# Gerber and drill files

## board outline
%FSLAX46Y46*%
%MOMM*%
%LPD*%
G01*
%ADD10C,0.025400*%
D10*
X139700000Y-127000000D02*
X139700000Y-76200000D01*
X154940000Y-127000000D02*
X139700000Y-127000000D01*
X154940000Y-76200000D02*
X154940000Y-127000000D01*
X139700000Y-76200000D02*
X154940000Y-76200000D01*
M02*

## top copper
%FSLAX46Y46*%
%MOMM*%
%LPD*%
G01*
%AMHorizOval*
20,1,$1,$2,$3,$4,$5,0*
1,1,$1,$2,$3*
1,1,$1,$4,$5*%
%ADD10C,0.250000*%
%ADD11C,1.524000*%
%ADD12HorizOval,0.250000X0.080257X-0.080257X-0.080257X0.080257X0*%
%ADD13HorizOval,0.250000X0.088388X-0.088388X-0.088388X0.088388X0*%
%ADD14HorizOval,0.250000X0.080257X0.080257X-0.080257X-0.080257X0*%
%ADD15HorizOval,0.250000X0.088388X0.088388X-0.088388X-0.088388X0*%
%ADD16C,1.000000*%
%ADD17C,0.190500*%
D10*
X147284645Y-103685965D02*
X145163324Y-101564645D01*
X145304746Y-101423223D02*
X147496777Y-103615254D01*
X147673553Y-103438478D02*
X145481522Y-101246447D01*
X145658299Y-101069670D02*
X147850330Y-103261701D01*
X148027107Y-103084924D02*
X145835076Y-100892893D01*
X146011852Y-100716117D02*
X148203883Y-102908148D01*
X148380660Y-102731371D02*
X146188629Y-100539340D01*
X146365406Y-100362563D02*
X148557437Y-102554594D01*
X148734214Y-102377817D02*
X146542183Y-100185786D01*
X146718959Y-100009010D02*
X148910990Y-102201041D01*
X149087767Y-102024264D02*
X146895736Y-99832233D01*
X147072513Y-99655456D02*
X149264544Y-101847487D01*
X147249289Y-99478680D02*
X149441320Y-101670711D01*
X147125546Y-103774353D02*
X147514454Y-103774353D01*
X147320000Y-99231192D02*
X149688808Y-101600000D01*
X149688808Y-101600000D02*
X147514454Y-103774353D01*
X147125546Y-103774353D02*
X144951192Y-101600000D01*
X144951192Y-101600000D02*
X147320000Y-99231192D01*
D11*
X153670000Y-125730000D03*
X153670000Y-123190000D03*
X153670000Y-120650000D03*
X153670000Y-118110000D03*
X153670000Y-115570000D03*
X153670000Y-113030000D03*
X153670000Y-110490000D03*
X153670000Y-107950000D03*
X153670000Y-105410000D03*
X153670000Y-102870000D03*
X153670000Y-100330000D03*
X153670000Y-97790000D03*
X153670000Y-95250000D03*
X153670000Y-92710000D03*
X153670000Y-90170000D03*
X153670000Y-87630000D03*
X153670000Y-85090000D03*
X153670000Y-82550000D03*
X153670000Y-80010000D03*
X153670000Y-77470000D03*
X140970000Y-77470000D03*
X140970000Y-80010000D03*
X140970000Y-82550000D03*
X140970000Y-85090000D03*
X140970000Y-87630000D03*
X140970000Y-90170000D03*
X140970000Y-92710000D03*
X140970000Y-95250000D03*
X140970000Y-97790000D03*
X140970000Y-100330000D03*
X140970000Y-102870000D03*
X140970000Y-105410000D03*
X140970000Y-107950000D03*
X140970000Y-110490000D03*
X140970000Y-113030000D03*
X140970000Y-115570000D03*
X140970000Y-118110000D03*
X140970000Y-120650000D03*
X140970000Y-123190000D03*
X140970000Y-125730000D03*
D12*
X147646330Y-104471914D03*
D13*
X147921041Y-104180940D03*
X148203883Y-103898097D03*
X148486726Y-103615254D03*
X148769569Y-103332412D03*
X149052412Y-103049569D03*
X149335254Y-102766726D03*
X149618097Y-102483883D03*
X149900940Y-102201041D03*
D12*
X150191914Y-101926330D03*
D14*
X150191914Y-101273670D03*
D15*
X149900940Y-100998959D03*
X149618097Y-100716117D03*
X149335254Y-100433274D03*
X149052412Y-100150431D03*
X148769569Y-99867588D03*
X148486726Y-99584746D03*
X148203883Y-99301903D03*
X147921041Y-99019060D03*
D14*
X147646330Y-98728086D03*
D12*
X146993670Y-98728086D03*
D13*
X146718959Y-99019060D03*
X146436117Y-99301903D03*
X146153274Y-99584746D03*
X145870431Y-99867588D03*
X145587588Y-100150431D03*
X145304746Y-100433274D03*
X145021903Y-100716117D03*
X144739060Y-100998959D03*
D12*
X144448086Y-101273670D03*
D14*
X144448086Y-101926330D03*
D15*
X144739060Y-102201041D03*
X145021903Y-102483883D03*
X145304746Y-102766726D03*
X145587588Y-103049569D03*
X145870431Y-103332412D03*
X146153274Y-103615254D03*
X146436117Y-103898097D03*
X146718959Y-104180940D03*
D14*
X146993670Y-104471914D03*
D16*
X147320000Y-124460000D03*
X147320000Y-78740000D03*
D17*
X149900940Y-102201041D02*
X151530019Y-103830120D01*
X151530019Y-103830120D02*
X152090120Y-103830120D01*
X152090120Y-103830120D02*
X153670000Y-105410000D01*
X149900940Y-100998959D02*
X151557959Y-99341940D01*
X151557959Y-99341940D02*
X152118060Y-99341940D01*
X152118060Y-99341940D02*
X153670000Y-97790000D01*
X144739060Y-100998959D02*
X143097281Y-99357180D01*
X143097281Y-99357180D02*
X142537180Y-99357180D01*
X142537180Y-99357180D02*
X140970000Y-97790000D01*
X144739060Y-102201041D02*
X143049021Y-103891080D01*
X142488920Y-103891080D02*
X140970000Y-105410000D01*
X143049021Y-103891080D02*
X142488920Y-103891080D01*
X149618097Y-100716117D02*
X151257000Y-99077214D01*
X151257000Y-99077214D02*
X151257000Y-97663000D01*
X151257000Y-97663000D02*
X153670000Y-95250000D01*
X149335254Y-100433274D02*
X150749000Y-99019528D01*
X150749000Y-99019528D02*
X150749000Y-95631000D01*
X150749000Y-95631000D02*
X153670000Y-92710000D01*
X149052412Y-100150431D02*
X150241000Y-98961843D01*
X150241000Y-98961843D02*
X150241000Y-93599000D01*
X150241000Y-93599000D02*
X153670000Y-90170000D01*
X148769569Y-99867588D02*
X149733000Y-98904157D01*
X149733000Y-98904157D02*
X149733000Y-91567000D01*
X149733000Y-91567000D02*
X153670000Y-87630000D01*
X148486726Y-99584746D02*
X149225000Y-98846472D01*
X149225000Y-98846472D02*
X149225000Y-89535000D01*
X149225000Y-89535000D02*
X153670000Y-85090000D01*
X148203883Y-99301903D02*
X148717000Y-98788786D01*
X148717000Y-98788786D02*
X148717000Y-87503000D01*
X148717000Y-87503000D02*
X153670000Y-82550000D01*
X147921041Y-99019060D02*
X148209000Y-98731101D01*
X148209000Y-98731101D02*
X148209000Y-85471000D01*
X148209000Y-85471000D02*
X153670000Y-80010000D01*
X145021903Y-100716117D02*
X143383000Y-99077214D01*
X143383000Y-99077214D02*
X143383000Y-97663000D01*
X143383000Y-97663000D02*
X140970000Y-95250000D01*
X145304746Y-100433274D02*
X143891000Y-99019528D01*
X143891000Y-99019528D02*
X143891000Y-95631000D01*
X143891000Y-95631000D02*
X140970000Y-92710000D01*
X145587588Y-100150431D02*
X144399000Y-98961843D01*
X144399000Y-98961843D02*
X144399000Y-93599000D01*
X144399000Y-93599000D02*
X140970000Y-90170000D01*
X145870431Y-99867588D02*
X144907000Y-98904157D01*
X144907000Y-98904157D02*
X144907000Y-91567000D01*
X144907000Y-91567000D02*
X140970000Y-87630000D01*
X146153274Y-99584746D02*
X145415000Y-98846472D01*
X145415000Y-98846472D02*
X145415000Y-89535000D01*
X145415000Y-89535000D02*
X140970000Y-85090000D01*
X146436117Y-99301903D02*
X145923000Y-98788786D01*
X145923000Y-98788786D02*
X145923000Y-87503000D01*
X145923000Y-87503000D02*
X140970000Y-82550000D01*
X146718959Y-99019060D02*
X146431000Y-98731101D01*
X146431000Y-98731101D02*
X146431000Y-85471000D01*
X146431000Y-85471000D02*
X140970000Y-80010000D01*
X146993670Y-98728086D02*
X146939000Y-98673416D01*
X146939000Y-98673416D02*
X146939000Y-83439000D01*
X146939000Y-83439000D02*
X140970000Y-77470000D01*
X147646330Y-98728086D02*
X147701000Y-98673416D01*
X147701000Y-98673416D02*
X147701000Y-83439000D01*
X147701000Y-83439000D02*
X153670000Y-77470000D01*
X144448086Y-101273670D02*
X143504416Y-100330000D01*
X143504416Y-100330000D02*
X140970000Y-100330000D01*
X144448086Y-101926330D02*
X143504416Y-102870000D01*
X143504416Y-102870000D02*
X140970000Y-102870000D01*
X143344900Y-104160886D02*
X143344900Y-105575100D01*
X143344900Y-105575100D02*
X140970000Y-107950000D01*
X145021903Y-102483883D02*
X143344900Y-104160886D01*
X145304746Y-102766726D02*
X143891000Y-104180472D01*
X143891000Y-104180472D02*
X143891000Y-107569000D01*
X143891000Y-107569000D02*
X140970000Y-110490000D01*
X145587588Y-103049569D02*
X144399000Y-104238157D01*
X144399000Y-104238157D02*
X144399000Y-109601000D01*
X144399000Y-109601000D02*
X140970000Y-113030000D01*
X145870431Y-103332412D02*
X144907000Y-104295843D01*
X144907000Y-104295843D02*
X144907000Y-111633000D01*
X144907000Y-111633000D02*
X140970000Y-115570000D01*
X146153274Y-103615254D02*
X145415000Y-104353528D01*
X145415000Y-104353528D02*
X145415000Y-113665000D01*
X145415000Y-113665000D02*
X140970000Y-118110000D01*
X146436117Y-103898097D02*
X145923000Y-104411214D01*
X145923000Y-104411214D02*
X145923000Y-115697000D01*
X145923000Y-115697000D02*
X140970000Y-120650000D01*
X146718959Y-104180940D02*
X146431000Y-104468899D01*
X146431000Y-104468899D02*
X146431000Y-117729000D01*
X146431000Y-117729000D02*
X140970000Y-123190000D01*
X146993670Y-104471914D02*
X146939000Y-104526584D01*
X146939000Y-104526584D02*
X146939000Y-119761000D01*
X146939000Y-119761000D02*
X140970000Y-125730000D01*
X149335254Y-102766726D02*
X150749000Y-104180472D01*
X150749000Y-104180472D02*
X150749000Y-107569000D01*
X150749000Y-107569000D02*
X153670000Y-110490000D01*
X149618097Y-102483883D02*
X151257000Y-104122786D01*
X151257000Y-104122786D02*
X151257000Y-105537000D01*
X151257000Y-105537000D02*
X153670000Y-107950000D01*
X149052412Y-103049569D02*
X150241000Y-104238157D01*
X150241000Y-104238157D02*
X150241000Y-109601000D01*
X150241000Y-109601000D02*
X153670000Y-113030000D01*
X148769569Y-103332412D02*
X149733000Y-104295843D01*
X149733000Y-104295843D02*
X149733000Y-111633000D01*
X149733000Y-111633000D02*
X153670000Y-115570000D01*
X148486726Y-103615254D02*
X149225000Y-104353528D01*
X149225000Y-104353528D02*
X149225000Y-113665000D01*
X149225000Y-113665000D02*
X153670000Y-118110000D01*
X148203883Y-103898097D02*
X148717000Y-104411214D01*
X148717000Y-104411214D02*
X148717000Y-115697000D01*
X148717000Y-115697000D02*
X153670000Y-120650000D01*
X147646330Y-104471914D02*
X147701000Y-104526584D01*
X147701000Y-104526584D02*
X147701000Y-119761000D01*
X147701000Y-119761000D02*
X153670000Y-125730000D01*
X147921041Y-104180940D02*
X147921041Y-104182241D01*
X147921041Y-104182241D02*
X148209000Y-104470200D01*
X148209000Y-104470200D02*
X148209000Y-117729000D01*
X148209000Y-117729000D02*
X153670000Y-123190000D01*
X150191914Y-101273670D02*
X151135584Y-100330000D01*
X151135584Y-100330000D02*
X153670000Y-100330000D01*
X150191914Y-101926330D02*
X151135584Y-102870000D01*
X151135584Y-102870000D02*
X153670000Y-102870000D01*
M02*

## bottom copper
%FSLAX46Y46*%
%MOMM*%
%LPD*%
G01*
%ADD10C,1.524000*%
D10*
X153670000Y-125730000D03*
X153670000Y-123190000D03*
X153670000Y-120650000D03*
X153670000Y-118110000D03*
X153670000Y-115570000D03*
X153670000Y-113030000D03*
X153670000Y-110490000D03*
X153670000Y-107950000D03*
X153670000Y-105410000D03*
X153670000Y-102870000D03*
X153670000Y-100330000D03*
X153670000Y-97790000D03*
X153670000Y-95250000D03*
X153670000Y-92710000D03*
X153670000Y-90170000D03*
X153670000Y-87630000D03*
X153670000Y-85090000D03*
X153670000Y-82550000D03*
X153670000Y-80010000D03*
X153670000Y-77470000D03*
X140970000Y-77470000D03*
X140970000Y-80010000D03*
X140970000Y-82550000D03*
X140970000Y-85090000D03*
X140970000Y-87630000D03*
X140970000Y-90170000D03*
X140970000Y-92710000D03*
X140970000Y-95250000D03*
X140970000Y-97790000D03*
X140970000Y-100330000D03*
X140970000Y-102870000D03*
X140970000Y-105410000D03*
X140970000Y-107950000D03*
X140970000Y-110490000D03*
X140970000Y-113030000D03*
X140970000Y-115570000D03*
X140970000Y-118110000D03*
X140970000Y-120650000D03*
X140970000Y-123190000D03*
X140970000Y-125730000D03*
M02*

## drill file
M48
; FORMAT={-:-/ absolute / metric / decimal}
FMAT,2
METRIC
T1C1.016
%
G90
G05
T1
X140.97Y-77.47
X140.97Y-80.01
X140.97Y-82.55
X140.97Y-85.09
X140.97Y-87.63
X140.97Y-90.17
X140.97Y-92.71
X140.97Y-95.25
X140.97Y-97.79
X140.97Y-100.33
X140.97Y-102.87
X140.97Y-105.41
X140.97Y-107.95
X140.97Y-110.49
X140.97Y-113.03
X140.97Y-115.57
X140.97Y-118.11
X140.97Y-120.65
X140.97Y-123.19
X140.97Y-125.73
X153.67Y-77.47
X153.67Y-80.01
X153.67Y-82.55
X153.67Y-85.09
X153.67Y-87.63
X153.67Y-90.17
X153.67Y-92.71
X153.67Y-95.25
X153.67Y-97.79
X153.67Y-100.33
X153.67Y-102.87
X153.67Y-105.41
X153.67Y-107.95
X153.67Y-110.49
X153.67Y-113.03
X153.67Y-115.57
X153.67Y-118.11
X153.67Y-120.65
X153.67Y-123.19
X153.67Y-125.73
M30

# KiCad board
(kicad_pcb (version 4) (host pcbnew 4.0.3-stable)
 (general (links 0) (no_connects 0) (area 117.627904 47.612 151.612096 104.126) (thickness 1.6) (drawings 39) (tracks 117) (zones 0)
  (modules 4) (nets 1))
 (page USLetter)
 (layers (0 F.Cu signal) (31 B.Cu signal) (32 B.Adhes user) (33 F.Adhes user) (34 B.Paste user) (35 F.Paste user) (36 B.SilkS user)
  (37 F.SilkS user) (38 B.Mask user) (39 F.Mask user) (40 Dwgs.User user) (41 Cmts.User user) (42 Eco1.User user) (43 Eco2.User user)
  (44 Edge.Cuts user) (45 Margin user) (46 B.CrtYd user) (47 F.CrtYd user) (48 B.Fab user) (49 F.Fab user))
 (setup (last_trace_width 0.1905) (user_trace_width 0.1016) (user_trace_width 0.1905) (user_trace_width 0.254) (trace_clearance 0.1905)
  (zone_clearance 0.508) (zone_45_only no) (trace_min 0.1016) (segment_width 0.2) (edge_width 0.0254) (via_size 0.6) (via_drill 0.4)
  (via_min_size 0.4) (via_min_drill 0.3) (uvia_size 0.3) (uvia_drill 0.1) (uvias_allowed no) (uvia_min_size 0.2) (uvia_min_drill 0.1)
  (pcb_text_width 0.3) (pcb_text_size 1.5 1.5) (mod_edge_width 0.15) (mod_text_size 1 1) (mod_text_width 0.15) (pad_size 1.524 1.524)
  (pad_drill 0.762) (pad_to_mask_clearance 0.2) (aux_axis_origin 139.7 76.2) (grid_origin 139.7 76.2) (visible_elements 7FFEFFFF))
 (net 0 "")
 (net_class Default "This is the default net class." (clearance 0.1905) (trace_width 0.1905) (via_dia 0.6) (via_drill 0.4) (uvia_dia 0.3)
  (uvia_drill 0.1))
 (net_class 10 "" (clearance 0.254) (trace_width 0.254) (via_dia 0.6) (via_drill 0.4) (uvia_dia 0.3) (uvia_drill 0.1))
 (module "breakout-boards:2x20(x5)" (layer F.Cu) (at 147.32 101.6)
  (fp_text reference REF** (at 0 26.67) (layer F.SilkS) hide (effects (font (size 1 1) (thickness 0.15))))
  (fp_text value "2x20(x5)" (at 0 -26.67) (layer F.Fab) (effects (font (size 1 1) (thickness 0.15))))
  (pad 1 thru_hole circle (at 6.35 24.13) (size 1.524 1.524) (drill 1.016) (layers *.Cu *.Mask))
  (pad 2 thru_hole circle (at 6.35 21.59) (size 1.524 1.524) (drill 1.016) (layers *.Cu *.Mask))
  (pad 3 thru_hole circle (at 6.35 19.05) (size 1.524 1.524) (drill 1.016) (layers *.Cu *.Mask))
  (pad 4 thru_hole circle (at 6.35 16.51) (size 1.524 1.524) (drill 1.016) (layers *.Cu *.Mask))
  (pad 5 thru_hole circle (at 6.35 13.97) (size 1.524 1.524) (drill 1.016) (layers *.Cu *.Mask))
  (pad 6 thru_hole circle (at 6.35 11.43) (size 1.524 1.524) (drill 1.016) (layers *.Cu *.Mask))
  (pad 7 thru_hole circle (at 6.35 8.89) (size 1.524 1.524) (drill 1.016) (layers *.Cu *.Mask))
  (pad 8 thru_hole circle (at 6.35 6.35) (size 1.524 1.524) (drill 1.016) (layers *.Cu *.Mask))
  (pad 9 thru_hole circle (at 6.35 3.81) (size 1.524 1.524) (drill 1.016) (layers *.Cu *.Mask))
  (pad 10 thru_hole circle (at 6.35 1.27) (size 1.524 1.524) (drill 1.016) (layers *.Cu *.Mask))
  (pad 11 thru_hole circle (at 6.35 -1.27) (size 1.524 1.524) (drill 1.016) (layers *.Cu *.Mask))
  (pad 12 thru_hole circle (at 6.35 -3.81) (size 1.524 1.524) (drill 1.016) (layers *.Cu *.Mask))
  (pad 13 thru_hole circle (at 6.35 -6.35) (size 1.524 1.524) (drill 1.016) (layers *.Cu *.Mask))
  (pad 14 thru_hole circle (at 6.35 -8.89) (size 1.524 1.524) (drill 1.016) (layers *.Cu *.Mask))
  (pad 15 thru_hole circle (at 6.35 -11.43) (size 1.524 1.524) (drill 1.016) (layers *.Cu *.Mask))
  (pad 16 thru_hole circle (at 6.35 -13.97) (size 1.524 1.524) (drill 1.016) (layers *.Cu *.Mask))
  (pad 17 thru_hole circle (at 6.35 -16.51) (size 1.524 1.524) (drill 1.016) (layers *.Cu *.Mask))
  (pad 18 thru_hole circle (at 6.35 -19.05) (size 1.524 1.524) (drill 1.016) (layers *.Cu *.Mask))
  (pad 19 thru_hole circle (at 6.35 -21.59) (size 1.524 1.524) (drill 1.016) (layers *.Cu *.Mask))
  (pad 20 thru_hole circle (at 6.35 -24.13) (size 1.524 1.524) (drill 1.016) (layers *.Cu *.Mask))
  (pad 21 thru_hole circle (at -6.35 -24.13) (size 1.524 1.524) (drill 1.016) (layers *.Cu *.Mask))
  (pad 22 thru_hole circle (at -6.35 -21.59) (size 1.524 1.524) (drill 1.016) (layers *.Cu *.Mask))
  (pad 23 thru_hole circle (at -6.35 -19.05) (size 1.524 1.524) (drill 1.016) (layers *.Cu *.Mask))
  (pad 24 thru_hole circle (at -6.35 -16.51) (size 1.524 1.524) (drill 1.016) (layers *.Cu *.Mask))
  (pad 25 thru_hole circle (at -6.35 -13.97) (size 1.524 1.524) (drill 1.016) (layers *.Cu *.Mask))
  (pad 26 thru_hole circle (at -6.35 -11.43) (size 1.524 1.524) (drill 1.016) (layers *.Cu *.Mask))
  (pad 27 thru_hole circle (at -6.35 -8.89) (size 1.524 1.524) (drill 1.016) (layers *.Cu *.Mask))
  (pad 28 thru_hole circle (at -6.35 -6.35) (size 1.524 1.524) (drill 1.016) (layers *.Cu *.Mask))
  (pad 29 thru_hole circle (at -6.35 -3.81) (size 1.524 1.524) (drill 1.016) (layers *.Cu *.Mask))
  (pad 30 thru_hole circle (at -6.35 -1.27) (size 1.524 1.524) (drill 1.016) (layers *.Cu *.Mask))
  (pad 31 thru_hole circle (at -6.35 1.27) (size 1.524 1.524) (drill 1.016) (layers *.Cu *.Mask))
  (pad 32 thru_hole circle (at -6.35 3.81) (size 1.524 1.524) (drill 1.016) (layers *.Cu *.Mask))
  (pad 33 thru_hole circle (at -6.35 6.35) (size 1.524 1.524) (drill 1.016) (layers *.Cu *.Mask))
  (pad 34 thru_hole circle (at -6.35 8.89) (size 1.524 1.524) (drill 1.016) (layers *.Cu *.Mask))
  (pad 35 thru_hole circle (at -6.35 11.43) (size 1.524 1.524) (drill 1.016) (layers *.Cu *.Mask))
  (pad 36 thru_hole circle (at -6.35 13.97) (size 1.524 1.524) (drill 1.016) (layers *.Cu *.Mask))
  (pad 37 thru_hole circle (at -6.35 16.51) (size 1.524 1.524) (drill 1.016) (layers *.Cu *.Mask))
  (pad 38 thru_hole circle (at -6.35 19.05) (size 1.524 1.524) (drill 1.016) (layers *.Cu *.Mask))
  (pad 39 thru_hole circle (at -6.35 21.59) (size 1.524 1.524) (drill 1.016) (layers *.Cu *.Mask))
  (pad 40 thru_hole circle (at -6.35 24.13) (size 1.524 1.524) (drill 1.016) (layers *.Cu *.Mask)))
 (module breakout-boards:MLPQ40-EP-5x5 (layer F.Cu) (at 147.32 101.6 315)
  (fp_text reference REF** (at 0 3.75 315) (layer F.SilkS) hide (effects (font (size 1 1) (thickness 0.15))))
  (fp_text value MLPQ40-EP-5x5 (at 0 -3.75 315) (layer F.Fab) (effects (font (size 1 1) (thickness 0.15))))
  (fp_line (start 1.45 1.5) (end -1.55 1.5) (layer F.Cu) (width 0.25))
  (fp_line (start -1.55 1.3) (end 1.55 1.3) (layer F.Cu) (width 0.25))
  (fp_line (start 1.55 1.05) (end -1.55 1.05) (layer F.Cu) (width 0.25))
  (fp_line (start -1.55 0.8) (end 1.55 0.8) (layer F.Cu) (width 0.25))
  (fp_line (start 1.55 0.55) (end -1.55 0.55) (layer F.Cu) (width 0.25))
  (fp_line (start -1.55 0.3) (end 1.55 0.3) (layer F.Cu) (width 0.25))
  (fp_line (start 1.55 0.05) (end -1.55 0.05) (layer F.Cu) (width 0.25))
  (fp_line (start -1.55 -0.2) (end 1.55 -0.2) (layer F.Cu) (width 0.25))
  (fp_line (start 1.55 -0.45) (end -1.55 -0.45) (layer F.Cu) (width 0.25))
  (fp_line (start -1.55 -0.7) (end 1.55 -0.7) (layer F.Cu) (width 0.25))
  (fp_line (start 1.55 -0.95) (end -1.55 -0.95) (layer F.Cu) (width 0.25))
  (fp_line (start -1.55 -1.2) (end 1.55 -1.2) (layer F.Cu) (width 0.25))
  (fp_line (start -1.55 -1.45) (end 1.55 -1.45) (layer F.Cu) (width 0.25))
  (fp_line (start 1.4 1.675) (end 1.675 1.4) (layer F.Cu) (width 0.25))
  (fp_line (start -1.675 -1.675) (end 1.675 -1.675) (layer F.Cu) (width 0.25))
  (fp_line (start 1.675 -1.675) (end 1.675 1.4) (layer F.Cu) (width 0.25))
  (fp_line (start 1.4 1.675) (end -1.675 1.675) (layer F.Cu) (width 0.25))
  (fp_line (start -1.675 1.675) (end -1.675 -1.675) (layer F.Cu) (width 0.25))
  (pad 1 smd oval (at 2.2615 1.8 315) (size 0.477 0.25) (layers F.Cu F.Paste F.Mask))
  (pad 2 smd oval (at 2.25 1.4 315) (size 0.5 0.25) (layers F.Cu F.Paste F.Mask))
  (pad 3 smd oval (at 2.25 1 315) (size 0.5 0.25) (layers F.Cu F.Paste F.Mask))
  (pad 4 smd oval (at 2.25 0.6 315) (size 0.5 0.25) (layers F.Cu F.Paste F.Mask))
  (pad 5 smd oval (at 2.25 0.2 315) (size 0.5 0.25) (layers F.Cu F.Paste F.Mask))
  (pad 6 smd oval (at 2.25 -0.2 315) (size 0.5 0.25) (layers F.Cu F.Paste F.Mask))
  (pad 7 smd oval (at 2.25 -0.6 315) (size 0.5 0.25) (layers F.Cu F.Paste F.Mask))
  (pad 8 smd oval (at 2.25 -1 315) (size 0.5 0.25) (layers F.Cu F.Paste F.Mask))
  (pad 9 smd oval (at 2.25 -1.4 315) (size 0.5 0.25) (layers F.Cu F.Paste F.Mask))
  (pad 10 smd oval (at 2.2615 -1.8 315) (size 0.477 0.25) (layers F.Cu F.Paste F.Mask))
  (pad 11 smd oval (at 1.8 -2.2615 45) (size 0.477 0.25) (layers F.Cu F.Paste F.Mask))
  (pad 12 smd oval (at 1.4 -2.25 45) (size 0.5 0.25) (layers F.Cu F.Paste F.Mask))
  (pad 13 smd oval (at 1 -2.25 45) (size 0.5 0.25) (layers F.Cu F.Paste F.Mask))
  (pad 14 smd oval (at 0.6 -2.25 45) (size 0.5 0.25) (layers F.Cu F.Paste F.Mask))
  (pad 15 smd oval (at 0.2 -2.25 45) (size 0.5 0.25) (layers F.Cu F.Paste F.Mask))
  (pad 16 smd oval (at -0.2 -2.25 45) (size 0.5 0.25) (layers F.Cu F.Paste F.Mask))
  (pad 17 smd oval (at -0.6 -2.25 45) (size 0.5 0.25) (layers F.Cu F.Paste F.Mask))
  (pad 18 smd oval (at -1 -2.25 45) (size 0.5 0.25) (layers F.Cu F.Paste F.Mask))
  (pad 19 smd oval (at -1.4 -2.25 45) (size 0.5 0.25) (layers F.Cu F.Paste F.Mask))
  (pad 20 smd oval (at -1.8 -2.2615 45) (size 0.477 0.25) (layers F.Cu F.Paste F.Mask))
  (pad 21 smd oval (at -2.2615 -1.8 315) (size 0.477 0.25) (layers F.Cu F.Paste F.Mask))
  (pad 22 smd oval (at -2.25 -1.4 315) (size 0.5 0.25) (layers F.Cu F.Paste F.Mask))
  (pad 23 smd oval (at -2.25 -1 315) (size 0.5 0.25) (layers F.Cu F.Paste F.Mask))
  (pad 24 smd oval (at -2.25 -0.6 315) (size 0.5 0.25) (layers F.Cu F.Paste F.Mask))
  (pad 25 smd oval (at -2.25 -0.2 315) (size 0.5 0.25) (layers F.Cu F.Paste F.Mask))
  (pad 26 smd oval (at -2.25 0.2 315) (size 0.5 0.25) (layers F.Cu F.Paste F.Mask))
  (pad 27 smd oval (at -2.25 0.6 315) (size 0.5 0.25) (layers F.Cu F.Paste F.Mask))
  (pad 28 smd oval (at -2.25 1 315) (size 0.5 0.25) (layers F.Cu F.Paste F.Mask))
  (pad 29 smd oval (at -2.25 1.4 315) (size 0.5 0.25) (layers F.Cu F.Paste F.Mask))
  (pad 30 smd oval (at -2.2615 1.8 315) (size 0.477 0.25) (layers F.Cu F.Paste F.Mask))
  (pad 31 smd oval (at -1.8 2.2615 45) (size 0.477 0.25) (layers F.Cu F.Paste F.Mask))
  (pad 32 smd oval (at -1.4 2.25 45) (size 0.5 0.25) (layers F.Cu F.Paste F.Mask))
  (pad 33 smd oval (at -1 2.25 45) (size 0.5 0.25) (layers F.Cu F.Paste F.Mask))
  (pad 34 smd oval (at -0.6 2.25 45) (size 0.5 0.25) (layers F.Cu F.Paste F.Mask))
  (pad 35 smd oval (at -0.2 2.25 45) (size 0.5 0.25) (layers F.Cu F.Paste F.Mask))
  (pad 36 smd oval (at 0.2 2.25 45) (size 0.5 0.25) (layers F.Cu F.Paste F.Mask))
  (pad 37 smd oval (at 0.6 2.25 45) (size 0.5 0.25) (layers F.Cu F.Paste F.Mask))
  (pad 38 smd oval (at 1 2.25 45) (size 0.5 0.25) (layers F.Cu F.Paste F.Mask))
  (pad 39 smd oval (at 1.4 2.25 45) (size 0.5 0.25) (layers F.Cu F.Paste F.Mask))
  (pad 40 smd oval (at 1.8 2.2615 45) (size 0.477 0.25) (layers F.Cu F.Paste F.Mask)))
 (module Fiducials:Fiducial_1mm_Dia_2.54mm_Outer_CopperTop (layer F.Cu) (at 147.32 124.46)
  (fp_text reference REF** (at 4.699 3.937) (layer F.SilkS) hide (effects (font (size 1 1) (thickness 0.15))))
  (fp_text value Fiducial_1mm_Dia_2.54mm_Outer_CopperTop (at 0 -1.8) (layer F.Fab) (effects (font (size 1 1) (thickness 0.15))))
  (pad ~ smd circle (at 0 0) (size 1 1) (layers F.Cu F.Mask) (solder_mask_margin 0.77) (clearance 0.77)))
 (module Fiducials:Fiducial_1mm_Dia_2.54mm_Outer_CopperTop (layer F.Cu) (at 147.32 78.74)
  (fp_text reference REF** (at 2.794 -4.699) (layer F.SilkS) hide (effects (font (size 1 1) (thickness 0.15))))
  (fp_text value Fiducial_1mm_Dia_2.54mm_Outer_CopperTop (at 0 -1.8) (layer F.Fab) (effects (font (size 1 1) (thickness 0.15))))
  (pad ~ smd circle (at 0 0) (size 1 1) (layers F.Cu F.Mask) (solder_mask_margin 0.77) (clearance 0.77)))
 (gr_line (start 139.7 127) (end 139.7 76.2) (angle 90) (layer Edge.Cuts) (width 0.0254))
 (gr_line (start 154.94 127) (end 139.7 127) (angle 90) (layer Edge.Cuts) (width 0.0254))
 (gr_line (start 154.94 76.2) (end 154.94 127) (angle 90) (layer Edge.Cuts) (width 0.0254))
 (gr_line (start 139.7 76.2) (end 154.94 76.2) (angle 90) (layer Edge.Cuts) (width 0.0254))
 (segment (start 149.90094 102.201041) (end 151.530019 103.83012) (width 0.1905) (layer F.Cu) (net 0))
 (segment (start 151.530019 103.83012) (end 152.09012 103.83012) (width 0.1905) (layer F.Cu) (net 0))
 (segment (start 152.09012 103.83012) (end 153.67 105.41) (width 0.1905) (layer F.Cu) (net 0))
 (segment (start 149.90094 100.998959) (end 151.557959 99.34194) (width 0.1905) (layer F.Cu) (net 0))
 (segment (start 151.557959 99.34194) (end 152.11806 99.34194) (width 0.1905) (layer F.Cu) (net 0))
 (segment (start 152.11806 99.34194) (end 153.67 97.79) (width 0.1905) (layer F.Cu) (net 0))
 (segment (start 144.73906 100.998959) (end 143.097281 99.35718) (width 0.1905) (layer F.Cu) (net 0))
 (segment (start 143.097281 99.35718) (end 142.53718 99.35718) (width 0.1905) (layer F.Cu) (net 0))
 (segment (start 142.53718 99.35718) (end 140.97 97.79) (width 0.1905) (layer F.Cu) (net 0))
 (segment (start 144.73906 102.201041) (end 143.049021 103.89108) (width 0.1905) (layer F.Cu) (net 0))
 (segment (start 142.48892 103.89108) (end 140.97 105.41) (width 0.1905) (layer F.Cu) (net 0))
 (segment (start 143.049021 103.89108) (end 142.48892 103.89108) (width 0.1905) (layer F.Cu) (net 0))
 (segment (start 149.618097 100.716117) (end 151.257 99.077214) (width 0.1905) (layer F.Cu) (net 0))
 (segment (start 151.257 99.077214) (end 151.257 97.663) (width 0.1905) (layer F.Cu) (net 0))
 (segment (start 151.257 97.663) (end 153.67 95.25) (width 0.1905) (layer F.Cu) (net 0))
 (segment (start 149.335254 100.433274) (end 150.749 99.019528) (width 0.1905) (layer F.Cu) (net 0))
 (segment (start 150.749 99.019528) (end 150.749 95.631) (width 0.1905) (layer F.Cu) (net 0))
 (segment (start 150.749 95.631) (end 153.67 92.71) (width 0.1905) (layer F.Cu) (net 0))
 (segment (start 149.052412 100.150431) (end 150.241 98.961843) (width 0.1905) (layer F.Cu) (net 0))
 (segment (start 150.241 98.961843) (end 150.241 93.599) (width 0.1905) (layer F.Cu) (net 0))
 (segment (start 150.241 93.599) (end 153.67 90.17) (width 0.1905) (layer F.Cu) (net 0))
 (segment (start 148.769569 99.867588) (end 149.733 98.904157) (width 0.1905) (layer F.Cu) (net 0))
 (segment (start 149.733 98.904157) (end 149.733 91.567) (width 0.1905) (layer F.Cu) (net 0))
 (segment (start 149.733 91.567) (end 153.67 87.63) (width 0.1905) (layer F.Cu) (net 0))
 (segment (start 148.486726 99.584746) (end 149.225 98.846472) (width 0.1905) (layer F.Cu) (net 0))
 (segment (start 149.225 98.846472) (end 149.225 89.535) (width 0.1905) (layer F.Cu) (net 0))
 (segment (start 149.225 89.535) (end 153.67 85.09) (width 0.1905) (layer F.Cu) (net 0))
 (segment (start 148.203883 99.301903) (end 148.717 98.788786) (width 0.1905) (layer F.Cu) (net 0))
 (segment (start 148.717 98.788786) (end 148.717 87.503) (width 0.1905) (layer F.Cu) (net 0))
 (segment (start 148.717 87.503) (end 153.67 82.55) (width 0.1905) (layer F.Cu) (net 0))
 (segment (start 147.921041 99.01906) (end 148.209 98.731101) (width 0.1905) (layer F.Cu) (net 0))
 (segment (start 148.209 98.731101) (end 148.209 85.471) (width 0.1905) (layer F.Cu) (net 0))
 (segment (start 148.209 85.471) (end 153.67 80.01) (width 0.1905) (layer F.Cu) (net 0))
 (segment (start 145.021903 100.716117) (end 143.383 99.077214) (width 0.1905) (layer F.Cu) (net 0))
 (segment (start 143.383 99.077214) (end 143.383 97.663) (width 0.1905) (layer F.Cu) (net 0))
 (segment (start 143.383 97.663) (end 140.97 95.25) (width 0.1905) (layer F.Cu) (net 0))
 (segment (start 145.304746 100.433274) (end 143.891 99.019528) (width 0.1905) (layer F.Cu) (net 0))
 (segment (start 143.891 99.019528) (end 143.891 95.631) (width 0.1905) (layer F.Cu) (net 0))
 (segment (start 143.891 95.631) (end 140.97 92.71) (width 0.1905) (layer F.Cu) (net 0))
 (segment (start 145.587588 100.150431) (end 144.399 98.961843) (width 0.1905) (layer F.Cu) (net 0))
 (segment (start 144.399 98.961843) (end 144.399 93.599) (width 0.1905) (layer F.Cu) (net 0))
 (segment (start 144.399 93.599) (end 140.97 90.17) (width 0.1905) (layer F.Cu) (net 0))
 (segment (start 145.870431 99.867588) (end 144.907 98.904157) (width 0.1905) (layer F.Cu) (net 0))
 (segment (start 144.907 98.904157) (end 144.907 91.567) (width 0.1905) (layer F.Cu) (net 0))
 (segment (start 144.907 91.567) (end 140.97 87.63) (width 0.1905) (layer F.Cu) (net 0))
 (segment (start 146.153274 99.584746) (end 145.415 98.846472) (width 0.1905) (layer F.Cu) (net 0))
 (segment (start 145.415 98.846472) (end 145.415 89.535) (width 0.1905) (layer F.Cu) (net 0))
 (segment (start 145.415 89.535) (end 140.97 85.09) (width 0.1905) (layer F.Cu) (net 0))
 (segment (start 146.436117 99.301903) (end 145.923 98.788786) (width 0.1905) (layer F.Cu) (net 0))
 (segment (start 145.923 98.788786) (end 145.923 87.503) (width 0.1905) (layer F.Cu) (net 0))
 (segment (start 145.923 87.503) (end 140.97 82.55) (width 0.1905) (layer F.Cu) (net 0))
 (segment (start 146.718959 99.01906) (end 146.431 98.731101) (width 0.1905) (layer F.Cu) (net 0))
 (segment (start 146.431 98.731101) (end 146.431 85.471) (width 0.1905) (layer F.Cu) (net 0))
 (segment (start 146.431 85.471) (end 140.97 80.01) (width 0.1905) (layer F.Cu) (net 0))
 (segment (start 146.99367 98.728086) (end 146.939 98.673416) (width 0.1905) (layer F.Cu) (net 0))
 (segment (start 146.939 98.673416) (end 146.939 83.439) (width 0.1905) (layer F.Cu) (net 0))
 (segment (start 146.939 83.439) (end 140.97 77.47) (width 0.1905) (layer F.Cu) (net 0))
 (segment (start 147.64633 98.728086) (end 147.701 98.673416) (width 0.1905) (layer F.Cu) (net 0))
 (segment (start 147.701 98.673416) (end 147.701 83.439) (width 0.1905) (layer F.Cu) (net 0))
 (segment (start 147.701 83.439) (end 153.67 77.47) (width 0.1905) (layer F.Cu) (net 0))
 (segment (start 144.448086 101.27367) (end 143.504416 100.33) (width 0.1905) (layer F.Cu) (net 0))
 (segment (start 143.504416 100.33) (end 140.97 100.33) (width 0.1905) (layer F.Cu) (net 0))
 (segment (start 144.448086 101.92633) (end 143.504416 102.87) (width 0.1905) (layer F.Cu) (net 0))
 (segment (start 143.504416 102.87) (end 140.97 102.87) (width 0.1905) (layer F.Cu) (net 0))
 (segment (start 143.3449 104.160886) (end 143.3449 105.5751) (width 0.1905) (layer F.Cu) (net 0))
 (segment (start 143.3449 105.5751) (end 140.97 107.95) (width 0.1905) (layer F.Cu) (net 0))
 (segment (start 145.021903 102.483883) (end 143.3449 104.160886) (width 0.1905) (layer F.Cu) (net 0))
 (segment (start 145.304746 102.766726) (end 143.891 104.180472) (width 0.1905) (layer F.Cu) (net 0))
 (segment (start 143.891 104.180472) (end 143.891 107.569) (width 0.1905) (layer F.Cu) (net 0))
 (segment (start 143.891 107.569) (end 140.97 110.49) (width 0.1905) (layer F.Cu) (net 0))
 (segment (start 145.587588 103.049569) (end 144.399 104.238157) (width 0.1905) (layer F.Cu) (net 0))
 (segment (start 144.399 104.238157) (end 144.399 109.601) (width 0.1905) (layer F.Cu) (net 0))
 (segment (start 144.399 109.601) (end 140.97 113.03) (width 0.1905) (layer F.Cu) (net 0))
 (segment (start 145.870431 103.332412) (end 144.907 104.295843) (width 0.1905) (layer F.Cu) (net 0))
 (segment (start 144.907 104.295843) (end 144.907 111.633) (width 0.1905) (layer F.Cu) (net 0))
 (segment (start 144.907 111.633) (end 140.97 115.57) (width 0.1905) (layer F.Cu) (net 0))
 (segment (start 146.153274 103.615254) (end 145.415 104.353528) (width 0.1905) (layer F.Cu) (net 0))
 (segment (start 145.415 104.353528) (end 145.415 113.665) (width 0.1905) (layer F.Cu) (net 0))
 (segment (start 145.415 113.665) (end 140.97 118.11) (width 0.1905) (layer F.Cu) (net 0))
 (segment (start 146.436117 103.898097) (end 145.923 104.411214) (width 0.1905) (layer F.Cu) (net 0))
 (segment (start 145.923 104.411214) (end 145.923 115.697) (width 0.1905) (layer F.Cu) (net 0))
 (segment (start 145.923 115.697) (end 140.97 120.65) (width 0.1905) (layer F.Cu) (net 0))
 (segment (start 146.718959 104.18094) (end 146.431 104.468899) (width 0.1905) (layer F.Cu) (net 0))
 (segment (start 146.431 104.468899) (end 146.431 117.729) (width 0.1905) (layer F.Cu) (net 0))
 (segment (start 146.431 117.729) (end 140.97 123.19) (width 0.1905) (layer F.Cu) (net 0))
 (segment (start 146.99367 104.471914) (end 146.939 104.526584) (width 0.1905) (layer F.Cu) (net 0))
 (segment (start 146.939 104.526584) (end 146.939 119.761) (width 0.1905) (layer F.Cu) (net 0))
 (segment (start 146.939 119.761) (end 140.97 125.73) (width 0.1905) (layer F.Cu) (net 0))
 (segment (start 149.335254 102.766726) (end 150.749 104.180472) (width 0.1905) (layer F.Cu) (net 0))
 (segment (start 150.749 104.180472) (end 150.749 107.569) (width 0.1905) (layer F.Cu) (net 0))
 (segment (start 150.749 107.569) (end 153.67 110.49) (width 0.1905) (layer F.Cu) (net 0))
 (segment (start 149.618097 102.483883) (end 151.257 104.122786) (width 0.1905) (layer F.Cu) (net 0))
 (segment (start 151.257 104.122786) (end 151.257 105.537) (width 0.1905) (layer F.Cu) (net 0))
 (segment (start 151.257 105.537) (end 153.67 107.95) (width 0.1905) (layer F.Cu) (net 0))
 (segment (start 149.052412 103.049569) (end 150.241 104.238157) (width 0.1905) (layer F.Cu) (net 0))
 (segment (start 150.241 104.238157) (end 150.241 109.601) (width 0.1905) (layer F.Cu) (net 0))
 (segment (start 150.241 109.601) (end 153.67 113.03) (width 0.1905) (layer F.Cu) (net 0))
 (segment (start 148.769569 103.332412) (end 149.733 104.295843) (width 0.1905) (layer F.Cu) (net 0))
 (segment (start 149.733 104.295843) (end 149.733 111.633) (width 0.1905) (layer F.Cu) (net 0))
 (segment (start 149.733 111.633) (end 153.67 115.57) (width 0.1905) (layer F.Cu) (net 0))
 (segment (start 148.486726 103.615254) (end 149.225 104.353528) (width 0.1905) (layer F.Cu) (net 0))
 (segment (start 149.225 104.353528) (end 149.225 113.665) (width 0.1905) (layer F.Cu) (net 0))
 (segment (start 149.225 113.665) (end 153.67 118.11) (width 0.1905) (layer F.Cu) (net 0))
 (segment (start 148.203883 103.898097) (end 148.717 104.411214) (width 0.1905) (layer F.Cu) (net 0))
 (segment (start 148.717 104.411214) (end 148.717 115.697) (width 0.1905) (layer F.Cu) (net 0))
 (segment (start 148.717 115.697) (end 153.67 120.65) (width 0.1905) (layer F.Cu) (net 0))
 (segment (start 147.64633 104.471914) (end 147.701 104.526584) (width 0.1905) (layer F.Cu) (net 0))
 (segment (start 147.701 104.526584) (end 147.701 119.761) (width 0.1905) (layer F.Cu) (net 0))
 (segment (start 147.701 119.761) (end 153.67 125.73) (width 0.1905) (layer F.Cu) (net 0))
 (segment (start 147.921041 104.18094) (end 147.921041 104.182241) (width 0.1905) (layer F.Cu) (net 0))
 (segment (start 147.921041 104.182241) (end 148.209 104.4702) (width 0.1905) (layer F.Cu) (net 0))
 (segment (start 148.209 104.4702) (end 148.209 117.729) (width 0.1905) (layer F.Cu) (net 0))
 (segment (start 148.209 117.729) (end 153.67 123.19) (width 0.1905) (layer F.Cu) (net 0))
 (segment (start 150.191914 101.27367) (end 151.135584 100.33) (width 0.1905) (layer F.Cu) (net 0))
 (segment (start 151.135584 100.33) (end 153.67 100.33) (width 0.1905) (layer F.Cu) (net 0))
 (segment (start 150.191914 101.92633) (end 151.135584 102.87) (width 0.1905) (layer F.Cu) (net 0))
 (segment (start 151.135584 102.87) (end 153.67 102.87) (width 0.1905) (layer F.Cu) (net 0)))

